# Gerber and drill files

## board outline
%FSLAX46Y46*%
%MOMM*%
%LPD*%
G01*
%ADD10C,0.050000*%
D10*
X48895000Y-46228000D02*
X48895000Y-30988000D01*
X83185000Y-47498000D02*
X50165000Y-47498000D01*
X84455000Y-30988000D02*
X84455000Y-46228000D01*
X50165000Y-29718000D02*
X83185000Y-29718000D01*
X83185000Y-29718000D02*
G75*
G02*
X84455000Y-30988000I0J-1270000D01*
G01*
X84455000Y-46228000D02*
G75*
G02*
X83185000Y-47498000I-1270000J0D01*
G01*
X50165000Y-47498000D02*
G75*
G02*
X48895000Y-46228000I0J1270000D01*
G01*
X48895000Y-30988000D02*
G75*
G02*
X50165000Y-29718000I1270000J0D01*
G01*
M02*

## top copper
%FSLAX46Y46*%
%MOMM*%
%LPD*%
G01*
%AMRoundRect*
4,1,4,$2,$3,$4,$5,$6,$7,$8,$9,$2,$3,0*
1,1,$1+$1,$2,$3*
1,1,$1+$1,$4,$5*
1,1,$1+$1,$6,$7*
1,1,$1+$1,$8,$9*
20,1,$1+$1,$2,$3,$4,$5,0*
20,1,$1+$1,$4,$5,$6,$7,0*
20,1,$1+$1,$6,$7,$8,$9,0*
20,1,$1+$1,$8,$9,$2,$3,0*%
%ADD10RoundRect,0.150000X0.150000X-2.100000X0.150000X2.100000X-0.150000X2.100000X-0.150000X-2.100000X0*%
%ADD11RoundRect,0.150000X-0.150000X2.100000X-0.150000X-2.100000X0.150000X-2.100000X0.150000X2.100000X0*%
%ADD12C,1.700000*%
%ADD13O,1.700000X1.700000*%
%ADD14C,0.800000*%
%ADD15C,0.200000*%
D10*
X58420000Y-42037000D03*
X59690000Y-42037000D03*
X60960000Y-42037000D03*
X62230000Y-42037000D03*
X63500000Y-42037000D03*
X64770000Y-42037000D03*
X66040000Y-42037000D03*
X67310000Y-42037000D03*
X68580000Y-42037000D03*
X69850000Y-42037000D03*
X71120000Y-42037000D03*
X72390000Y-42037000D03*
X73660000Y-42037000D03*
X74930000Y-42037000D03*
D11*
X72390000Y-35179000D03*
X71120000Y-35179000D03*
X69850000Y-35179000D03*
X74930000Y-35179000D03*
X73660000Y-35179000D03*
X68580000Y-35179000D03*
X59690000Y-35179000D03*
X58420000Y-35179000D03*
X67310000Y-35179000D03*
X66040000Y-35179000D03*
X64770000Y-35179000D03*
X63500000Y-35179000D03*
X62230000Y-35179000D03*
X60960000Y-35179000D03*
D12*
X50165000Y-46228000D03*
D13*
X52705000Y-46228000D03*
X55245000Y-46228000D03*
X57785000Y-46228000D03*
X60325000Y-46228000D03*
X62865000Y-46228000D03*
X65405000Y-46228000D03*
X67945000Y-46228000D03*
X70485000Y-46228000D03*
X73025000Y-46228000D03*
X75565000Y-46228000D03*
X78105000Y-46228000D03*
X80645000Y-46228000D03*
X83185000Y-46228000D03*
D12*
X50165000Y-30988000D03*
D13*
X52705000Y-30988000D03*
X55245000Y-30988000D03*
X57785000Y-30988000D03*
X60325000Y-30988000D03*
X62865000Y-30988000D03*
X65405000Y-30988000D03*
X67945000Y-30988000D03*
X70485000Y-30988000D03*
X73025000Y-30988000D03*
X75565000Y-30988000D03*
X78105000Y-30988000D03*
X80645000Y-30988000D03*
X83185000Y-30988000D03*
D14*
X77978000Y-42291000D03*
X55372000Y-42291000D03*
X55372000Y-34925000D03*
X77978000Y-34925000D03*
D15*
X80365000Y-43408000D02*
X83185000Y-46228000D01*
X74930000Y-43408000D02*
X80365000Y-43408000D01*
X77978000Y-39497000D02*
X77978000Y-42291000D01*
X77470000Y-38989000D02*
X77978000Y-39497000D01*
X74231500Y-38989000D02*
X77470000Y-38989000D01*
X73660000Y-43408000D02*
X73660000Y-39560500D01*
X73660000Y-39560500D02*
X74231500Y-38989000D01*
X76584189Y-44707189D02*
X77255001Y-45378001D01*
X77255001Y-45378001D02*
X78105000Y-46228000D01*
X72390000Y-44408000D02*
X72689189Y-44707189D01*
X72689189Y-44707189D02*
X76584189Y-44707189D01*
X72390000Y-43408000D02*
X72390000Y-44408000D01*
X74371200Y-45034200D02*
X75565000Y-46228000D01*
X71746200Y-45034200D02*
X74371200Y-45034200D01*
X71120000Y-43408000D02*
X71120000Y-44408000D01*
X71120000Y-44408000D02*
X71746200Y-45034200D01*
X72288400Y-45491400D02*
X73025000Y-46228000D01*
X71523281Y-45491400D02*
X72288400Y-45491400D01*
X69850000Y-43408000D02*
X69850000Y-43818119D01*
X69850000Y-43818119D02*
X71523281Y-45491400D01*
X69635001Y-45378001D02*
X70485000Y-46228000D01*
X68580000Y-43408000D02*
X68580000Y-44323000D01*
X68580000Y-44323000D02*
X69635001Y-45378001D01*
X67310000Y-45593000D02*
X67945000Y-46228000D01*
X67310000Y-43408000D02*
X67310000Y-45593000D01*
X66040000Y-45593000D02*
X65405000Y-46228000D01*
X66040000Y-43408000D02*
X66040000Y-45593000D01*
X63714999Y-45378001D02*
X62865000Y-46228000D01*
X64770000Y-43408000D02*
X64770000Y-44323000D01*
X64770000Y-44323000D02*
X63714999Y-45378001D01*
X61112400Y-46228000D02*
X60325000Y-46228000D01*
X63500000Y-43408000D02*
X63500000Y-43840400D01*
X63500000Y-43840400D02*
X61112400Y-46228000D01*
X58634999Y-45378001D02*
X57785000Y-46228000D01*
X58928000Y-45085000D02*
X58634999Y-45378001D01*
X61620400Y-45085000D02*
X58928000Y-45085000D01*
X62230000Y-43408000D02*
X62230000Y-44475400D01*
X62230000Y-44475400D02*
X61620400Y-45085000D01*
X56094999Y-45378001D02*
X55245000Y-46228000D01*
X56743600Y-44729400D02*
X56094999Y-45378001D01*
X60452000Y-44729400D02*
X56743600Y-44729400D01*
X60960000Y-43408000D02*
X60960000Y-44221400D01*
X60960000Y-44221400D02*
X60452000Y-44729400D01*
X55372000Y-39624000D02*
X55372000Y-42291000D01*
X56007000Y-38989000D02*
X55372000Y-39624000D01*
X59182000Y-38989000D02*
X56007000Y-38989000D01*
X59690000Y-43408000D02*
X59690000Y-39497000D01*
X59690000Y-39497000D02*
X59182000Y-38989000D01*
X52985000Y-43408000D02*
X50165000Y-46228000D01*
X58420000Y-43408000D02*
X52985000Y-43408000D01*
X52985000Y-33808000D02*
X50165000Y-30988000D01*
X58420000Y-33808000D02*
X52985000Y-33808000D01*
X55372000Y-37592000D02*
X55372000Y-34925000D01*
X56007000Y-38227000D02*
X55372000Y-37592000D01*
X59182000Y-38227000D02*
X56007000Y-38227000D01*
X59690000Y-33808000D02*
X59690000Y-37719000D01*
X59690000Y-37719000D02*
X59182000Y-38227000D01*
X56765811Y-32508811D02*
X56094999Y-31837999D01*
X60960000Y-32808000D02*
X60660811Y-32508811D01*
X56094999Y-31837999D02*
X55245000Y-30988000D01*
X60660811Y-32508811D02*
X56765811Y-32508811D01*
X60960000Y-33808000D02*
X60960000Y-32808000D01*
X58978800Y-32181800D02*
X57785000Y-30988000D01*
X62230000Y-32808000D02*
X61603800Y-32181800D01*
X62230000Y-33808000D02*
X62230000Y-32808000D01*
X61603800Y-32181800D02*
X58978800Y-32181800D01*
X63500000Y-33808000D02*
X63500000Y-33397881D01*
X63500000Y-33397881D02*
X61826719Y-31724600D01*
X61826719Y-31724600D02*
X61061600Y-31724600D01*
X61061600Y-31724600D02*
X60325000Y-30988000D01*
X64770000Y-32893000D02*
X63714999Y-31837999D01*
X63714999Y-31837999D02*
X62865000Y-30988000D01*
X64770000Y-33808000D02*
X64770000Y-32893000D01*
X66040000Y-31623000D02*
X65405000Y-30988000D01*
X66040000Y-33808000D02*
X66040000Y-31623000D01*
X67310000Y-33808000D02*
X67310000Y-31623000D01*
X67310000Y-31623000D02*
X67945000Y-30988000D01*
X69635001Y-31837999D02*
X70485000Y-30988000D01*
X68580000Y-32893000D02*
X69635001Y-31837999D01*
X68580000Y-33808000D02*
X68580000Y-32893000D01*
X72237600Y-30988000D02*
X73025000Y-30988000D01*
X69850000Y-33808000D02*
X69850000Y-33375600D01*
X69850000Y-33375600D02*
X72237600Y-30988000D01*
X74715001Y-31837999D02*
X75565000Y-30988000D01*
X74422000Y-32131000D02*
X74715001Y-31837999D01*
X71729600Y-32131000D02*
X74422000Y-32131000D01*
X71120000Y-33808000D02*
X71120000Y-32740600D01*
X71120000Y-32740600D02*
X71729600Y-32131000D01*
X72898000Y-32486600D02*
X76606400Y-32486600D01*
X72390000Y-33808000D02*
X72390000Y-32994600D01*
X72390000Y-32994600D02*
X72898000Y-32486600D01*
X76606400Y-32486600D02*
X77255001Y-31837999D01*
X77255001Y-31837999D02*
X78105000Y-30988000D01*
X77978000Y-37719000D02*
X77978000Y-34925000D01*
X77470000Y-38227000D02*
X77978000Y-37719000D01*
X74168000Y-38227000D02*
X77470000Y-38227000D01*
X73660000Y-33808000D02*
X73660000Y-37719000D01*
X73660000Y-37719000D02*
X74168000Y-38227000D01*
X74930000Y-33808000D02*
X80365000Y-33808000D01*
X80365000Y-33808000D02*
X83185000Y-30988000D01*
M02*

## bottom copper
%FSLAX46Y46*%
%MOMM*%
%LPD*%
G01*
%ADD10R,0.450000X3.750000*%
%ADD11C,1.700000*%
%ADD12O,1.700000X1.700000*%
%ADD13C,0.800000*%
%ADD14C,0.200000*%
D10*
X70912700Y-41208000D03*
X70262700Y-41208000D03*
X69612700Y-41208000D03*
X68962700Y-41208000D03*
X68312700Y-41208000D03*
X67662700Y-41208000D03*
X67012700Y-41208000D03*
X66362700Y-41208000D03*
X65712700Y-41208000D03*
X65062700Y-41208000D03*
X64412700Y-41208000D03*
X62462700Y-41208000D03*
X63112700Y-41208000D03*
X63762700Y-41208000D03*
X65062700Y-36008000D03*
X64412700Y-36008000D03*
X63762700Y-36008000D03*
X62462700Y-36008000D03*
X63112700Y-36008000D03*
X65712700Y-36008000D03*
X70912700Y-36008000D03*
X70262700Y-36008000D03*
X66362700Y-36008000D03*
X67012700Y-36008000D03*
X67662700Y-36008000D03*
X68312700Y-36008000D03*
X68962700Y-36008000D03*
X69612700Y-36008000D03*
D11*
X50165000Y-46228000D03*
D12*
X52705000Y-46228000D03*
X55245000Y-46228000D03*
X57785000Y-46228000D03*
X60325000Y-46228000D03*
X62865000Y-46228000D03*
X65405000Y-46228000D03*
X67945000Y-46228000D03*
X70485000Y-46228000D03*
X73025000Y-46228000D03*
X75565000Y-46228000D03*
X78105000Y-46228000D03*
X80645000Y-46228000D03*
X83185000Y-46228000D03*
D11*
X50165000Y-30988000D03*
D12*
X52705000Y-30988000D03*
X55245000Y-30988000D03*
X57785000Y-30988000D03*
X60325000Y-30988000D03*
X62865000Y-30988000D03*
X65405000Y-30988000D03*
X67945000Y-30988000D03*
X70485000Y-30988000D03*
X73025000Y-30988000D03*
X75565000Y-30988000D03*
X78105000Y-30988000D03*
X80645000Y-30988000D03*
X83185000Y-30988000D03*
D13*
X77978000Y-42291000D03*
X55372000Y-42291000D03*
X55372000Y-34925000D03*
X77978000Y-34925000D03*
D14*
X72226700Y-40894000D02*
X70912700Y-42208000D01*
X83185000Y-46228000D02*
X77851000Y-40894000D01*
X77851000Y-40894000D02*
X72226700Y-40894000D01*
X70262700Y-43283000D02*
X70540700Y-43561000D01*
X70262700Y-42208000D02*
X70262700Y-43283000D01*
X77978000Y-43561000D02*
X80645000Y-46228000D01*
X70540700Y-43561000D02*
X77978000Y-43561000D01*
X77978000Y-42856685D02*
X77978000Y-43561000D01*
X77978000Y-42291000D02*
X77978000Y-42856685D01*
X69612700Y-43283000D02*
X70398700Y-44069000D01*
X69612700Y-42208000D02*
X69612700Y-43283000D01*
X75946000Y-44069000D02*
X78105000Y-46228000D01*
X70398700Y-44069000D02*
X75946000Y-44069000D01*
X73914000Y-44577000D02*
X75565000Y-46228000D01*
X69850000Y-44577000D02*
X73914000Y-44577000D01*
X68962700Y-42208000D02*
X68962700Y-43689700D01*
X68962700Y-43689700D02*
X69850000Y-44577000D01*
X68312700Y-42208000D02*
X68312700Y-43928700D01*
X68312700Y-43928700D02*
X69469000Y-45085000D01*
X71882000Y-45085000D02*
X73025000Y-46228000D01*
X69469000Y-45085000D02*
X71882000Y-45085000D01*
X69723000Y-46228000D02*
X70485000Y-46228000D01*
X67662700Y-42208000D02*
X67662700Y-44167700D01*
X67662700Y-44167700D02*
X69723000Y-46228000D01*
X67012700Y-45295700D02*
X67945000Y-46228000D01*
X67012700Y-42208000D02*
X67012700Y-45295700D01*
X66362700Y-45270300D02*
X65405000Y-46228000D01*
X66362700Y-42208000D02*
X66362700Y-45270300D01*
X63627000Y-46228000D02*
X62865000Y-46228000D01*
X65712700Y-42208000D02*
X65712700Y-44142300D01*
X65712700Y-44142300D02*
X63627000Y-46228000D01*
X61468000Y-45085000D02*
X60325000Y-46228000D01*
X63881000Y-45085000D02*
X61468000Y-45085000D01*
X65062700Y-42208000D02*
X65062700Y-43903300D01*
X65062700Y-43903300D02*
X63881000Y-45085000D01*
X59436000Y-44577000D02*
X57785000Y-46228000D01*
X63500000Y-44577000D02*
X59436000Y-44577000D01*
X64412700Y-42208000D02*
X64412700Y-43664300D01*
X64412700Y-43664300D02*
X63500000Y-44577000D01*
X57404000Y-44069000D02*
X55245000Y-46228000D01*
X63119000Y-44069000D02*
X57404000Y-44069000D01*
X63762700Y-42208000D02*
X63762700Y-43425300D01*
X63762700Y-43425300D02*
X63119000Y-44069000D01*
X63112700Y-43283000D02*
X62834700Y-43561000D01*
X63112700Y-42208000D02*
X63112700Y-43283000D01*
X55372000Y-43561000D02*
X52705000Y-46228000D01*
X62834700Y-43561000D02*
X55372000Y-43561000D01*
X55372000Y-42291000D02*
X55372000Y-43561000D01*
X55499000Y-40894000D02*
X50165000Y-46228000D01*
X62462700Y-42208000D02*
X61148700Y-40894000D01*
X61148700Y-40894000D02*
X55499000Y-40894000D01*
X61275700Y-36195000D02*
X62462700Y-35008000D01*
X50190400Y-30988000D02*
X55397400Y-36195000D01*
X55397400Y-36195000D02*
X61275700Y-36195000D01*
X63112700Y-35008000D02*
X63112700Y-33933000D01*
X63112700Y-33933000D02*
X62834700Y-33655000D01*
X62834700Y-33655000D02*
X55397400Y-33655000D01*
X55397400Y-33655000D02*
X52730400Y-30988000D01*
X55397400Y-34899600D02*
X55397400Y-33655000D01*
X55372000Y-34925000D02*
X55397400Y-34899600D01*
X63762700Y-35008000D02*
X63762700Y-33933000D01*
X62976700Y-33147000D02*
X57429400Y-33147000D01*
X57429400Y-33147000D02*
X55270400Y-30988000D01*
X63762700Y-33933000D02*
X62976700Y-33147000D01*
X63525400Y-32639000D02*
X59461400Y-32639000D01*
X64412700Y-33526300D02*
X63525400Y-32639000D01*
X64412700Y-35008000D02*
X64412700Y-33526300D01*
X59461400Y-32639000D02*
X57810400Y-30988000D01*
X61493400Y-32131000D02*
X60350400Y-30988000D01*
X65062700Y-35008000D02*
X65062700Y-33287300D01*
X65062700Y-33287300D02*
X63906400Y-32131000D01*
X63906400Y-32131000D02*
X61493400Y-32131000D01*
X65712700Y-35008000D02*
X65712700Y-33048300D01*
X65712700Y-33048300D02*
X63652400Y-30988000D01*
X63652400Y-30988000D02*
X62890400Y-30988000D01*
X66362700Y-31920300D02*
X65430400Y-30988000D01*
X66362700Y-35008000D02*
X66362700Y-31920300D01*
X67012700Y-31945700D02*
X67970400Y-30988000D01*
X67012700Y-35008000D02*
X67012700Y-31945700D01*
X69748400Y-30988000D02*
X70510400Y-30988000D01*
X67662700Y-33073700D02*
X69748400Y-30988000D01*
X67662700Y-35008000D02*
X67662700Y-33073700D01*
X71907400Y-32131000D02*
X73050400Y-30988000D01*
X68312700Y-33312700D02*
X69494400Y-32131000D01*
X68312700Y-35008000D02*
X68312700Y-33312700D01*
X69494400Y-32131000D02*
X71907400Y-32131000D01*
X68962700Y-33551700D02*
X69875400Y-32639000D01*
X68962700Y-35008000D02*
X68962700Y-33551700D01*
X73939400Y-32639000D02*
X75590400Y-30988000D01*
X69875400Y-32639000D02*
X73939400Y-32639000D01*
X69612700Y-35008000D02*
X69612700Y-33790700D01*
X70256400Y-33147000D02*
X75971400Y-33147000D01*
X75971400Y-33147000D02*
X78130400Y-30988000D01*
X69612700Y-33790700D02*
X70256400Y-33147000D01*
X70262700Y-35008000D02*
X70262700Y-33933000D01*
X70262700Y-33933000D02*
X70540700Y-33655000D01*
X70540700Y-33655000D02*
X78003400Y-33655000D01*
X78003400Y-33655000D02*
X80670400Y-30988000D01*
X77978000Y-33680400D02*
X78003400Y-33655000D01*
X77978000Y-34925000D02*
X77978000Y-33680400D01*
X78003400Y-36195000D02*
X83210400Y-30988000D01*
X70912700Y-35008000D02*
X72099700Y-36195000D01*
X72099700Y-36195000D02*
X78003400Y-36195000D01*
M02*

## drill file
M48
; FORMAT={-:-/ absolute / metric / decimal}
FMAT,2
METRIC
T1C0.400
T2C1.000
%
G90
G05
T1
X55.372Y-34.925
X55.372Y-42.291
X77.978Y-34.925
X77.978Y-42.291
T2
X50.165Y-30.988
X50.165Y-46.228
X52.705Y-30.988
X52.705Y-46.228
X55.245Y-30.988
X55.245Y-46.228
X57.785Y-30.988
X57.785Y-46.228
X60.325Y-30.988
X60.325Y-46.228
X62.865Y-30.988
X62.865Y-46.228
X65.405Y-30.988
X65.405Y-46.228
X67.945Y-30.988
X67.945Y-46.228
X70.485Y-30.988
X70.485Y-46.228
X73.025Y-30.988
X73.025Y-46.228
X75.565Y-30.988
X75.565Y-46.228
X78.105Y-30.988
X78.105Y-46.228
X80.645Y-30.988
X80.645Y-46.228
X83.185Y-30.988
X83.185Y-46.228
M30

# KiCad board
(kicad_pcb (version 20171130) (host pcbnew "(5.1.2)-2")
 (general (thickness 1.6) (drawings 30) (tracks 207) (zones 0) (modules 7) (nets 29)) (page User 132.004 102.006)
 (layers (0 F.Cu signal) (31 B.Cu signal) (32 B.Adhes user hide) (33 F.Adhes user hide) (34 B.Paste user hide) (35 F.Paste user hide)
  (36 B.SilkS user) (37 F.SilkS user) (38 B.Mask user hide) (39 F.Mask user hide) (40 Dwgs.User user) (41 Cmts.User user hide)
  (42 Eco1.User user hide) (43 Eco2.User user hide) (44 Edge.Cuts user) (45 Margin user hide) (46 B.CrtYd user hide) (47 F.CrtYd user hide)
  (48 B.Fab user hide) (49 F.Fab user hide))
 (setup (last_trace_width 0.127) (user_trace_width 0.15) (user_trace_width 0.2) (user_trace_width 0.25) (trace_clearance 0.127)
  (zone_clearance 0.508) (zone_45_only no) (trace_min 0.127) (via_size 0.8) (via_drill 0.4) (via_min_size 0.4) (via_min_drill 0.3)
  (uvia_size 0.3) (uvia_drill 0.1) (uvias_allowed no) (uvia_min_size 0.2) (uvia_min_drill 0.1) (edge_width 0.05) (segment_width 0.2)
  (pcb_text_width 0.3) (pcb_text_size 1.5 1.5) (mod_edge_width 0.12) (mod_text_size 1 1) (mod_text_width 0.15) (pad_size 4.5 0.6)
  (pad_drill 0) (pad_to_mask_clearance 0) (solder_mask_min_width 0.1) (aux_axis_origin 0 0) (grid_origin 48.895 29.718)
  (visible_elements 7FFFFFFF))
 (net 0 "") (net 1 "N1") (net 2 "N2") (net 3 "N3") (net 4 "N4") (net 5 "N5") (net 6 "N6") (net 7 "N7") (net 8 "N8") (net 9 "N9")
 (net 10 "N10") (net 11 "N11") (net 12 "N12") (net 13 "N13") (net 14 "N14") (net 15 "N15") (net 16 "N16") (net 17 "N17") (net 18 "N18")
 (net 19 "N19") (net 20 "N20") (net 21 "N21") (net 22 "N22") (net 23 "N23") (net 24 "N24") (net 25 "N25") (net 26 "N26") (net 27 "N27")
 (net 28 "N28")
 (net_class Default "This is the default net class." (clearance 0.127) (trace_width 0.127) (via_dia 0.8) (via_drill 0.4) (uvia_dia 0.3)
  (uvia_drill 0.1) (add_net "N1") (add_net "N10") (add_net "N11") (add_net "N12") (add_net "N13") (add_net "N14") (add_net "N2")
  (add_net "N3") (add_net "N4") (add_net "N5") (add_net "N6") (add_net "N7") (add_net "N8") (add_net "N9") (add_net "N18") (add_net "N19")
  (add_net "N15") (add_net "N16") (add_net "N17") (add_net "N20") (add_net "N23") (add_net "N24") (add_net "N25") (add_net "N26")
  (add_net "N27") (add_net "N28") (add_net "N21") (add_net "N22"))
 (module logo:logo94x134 (layer B.Cu) (at 79.502 38.608 180)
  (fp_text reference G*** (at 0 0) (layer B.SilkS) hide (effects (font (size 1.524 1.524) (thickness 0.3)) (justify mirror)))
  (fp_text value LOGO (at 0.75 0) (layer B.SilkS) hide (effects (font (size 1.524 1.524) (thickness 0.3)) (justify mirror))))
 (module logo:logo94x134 (layer F.Cu) (at 52.705 38.608)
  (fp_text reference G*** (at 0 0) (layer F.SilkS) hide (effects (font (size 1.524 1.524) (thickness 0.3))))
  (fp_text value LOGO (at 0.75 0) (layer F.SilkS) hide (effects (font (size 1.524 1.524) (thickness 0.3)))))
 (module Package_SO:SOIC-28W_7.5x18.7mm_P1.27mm (layer F.Cu) (at 66.675 38.608 90)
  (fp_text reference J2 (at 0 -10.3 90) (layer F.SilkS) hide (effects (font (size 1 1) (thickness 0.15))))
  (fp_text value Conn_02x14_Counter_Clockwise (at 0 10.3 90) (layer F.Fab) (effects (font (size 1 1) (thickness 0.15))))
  (pad 1 smd roundrect (at -3.429 -8.255 90) (size 4.5 0.6) (layers F.Cu F.Paste F.Mask) (roundrect_rratio 0.25) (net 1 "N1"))
  (pad 2 smd roundrect (at -3.429 -6.985 90) (size 4.5 0.6) (layers F.Cu F.Paste F.Mask) (roundrect_rratio 0.25) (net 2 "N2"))
  (pad 3 smd roundrect (at -3.429 -5.715 90) (size 4.5 0.6) (layers F.Cu F.Paste F.Mask) (roundrect_rratio 0.25) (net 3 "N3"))
  (pad 4 smd roundrect (at -3.429 -4.445 90) (size 4.5 0.6) (layers F.Cu F.Paste F.Mask) (roundrect_rratio 0.25) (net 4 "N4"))
  (pad 5 smd roundrect (at -3.429 -3.175 90) (size 4.5 0.6) (layers F.Cu F.Paste F.Mask) (roundrect_rratio 0.25) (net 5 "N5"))
  (pad 6 smd roundrect (at -3.429 -1.905 90) (size 4.5 0.6) (layers F.Cu F.Paste F.Mask) (roundrect_rratio 0.25) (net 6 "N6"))
  (pad 7 smd roundrect (at -3.429 -0.635 90) (size 4.5 0.6) (layers F.Cu F.Paste F.Mask) (roundrect_rratio 0.25) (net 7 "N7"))
  (pad 8 smd roundrect (at -3.429 0.635 90) (size 4.5 0.6) (layers F.Cu F.Paste F.Mask) (roundrect_rratio 0.25) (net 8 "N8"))
  (pad 9 smd roundrect (at -3.429 1.905 90) (size 4.5 0.6) (layers F.Cu F.Paste F.Mask) (roundrect_rratio 0.25) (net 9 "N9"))
  (pad 10 smd roundrect (at -3.429 3.175 90) (size 4.5 0.6) (layers F.Cu F.Paste F.Mask) (roundrect_rratio 0.25) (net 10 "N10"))
  (pad 11 smd roundrect (at -3.429 4.445 90) (size 4.5 0.6) (layers F.Cu F.Paste F.Mask) (roundrect_rratio 0.25) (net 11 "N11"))
  (pad 12 smd roundrect (at -3.429 5.715 90) (size 4.5 0.6) (layers F.Cu F.Paste F.Mask) (roundrect_rratio 0.25) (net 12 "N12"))
  (pad 13 smd roundrect (at -3.429 6.985 90) (size 4.5 0.6) (layers F.Cu F.Paste F.Mask) (roundrect_rratio 0.25) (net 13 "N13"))
  (pad 14 smd roundrect (at -3.429 8.255 90) (size 4.5 0.6) (layers F.Cu F.Paste F.Mask) (roundrect_rratio 0.25) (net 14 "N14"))
  (pad 17 smd roundrect (at 3.429 5.715 270) (size 4.5 0.6) (layers F.Cu F.Paste F.Mask) (roundrect_rratio 0.25) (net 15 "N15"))
  (pad 18 smd roundrect (at 3.429 4.445 270) (size 4.5 0.6) (layers F.Cu F.Paste F.Mask) (roundrect_rratio 0.25) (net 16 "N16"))
  (pad 19 smd roundrect (at 3.429 3.175 270) (size 4.5 0.6) (layers F.Cu F.Paste F.Mask) (roundrect_rratio 0.25) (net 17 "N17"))
  (pad 15 smd roundrect (at 3.429 8.255 270) (size 4.5 0.6) (layers F.Cu F.Paste F.Mask) (roundrect_rratio 0.25) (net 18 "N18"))
  (pad 16 smd roundrect (at 3.429 6.985 270) (size 4.5 0.6) (layers F.Cu F.Paste F.Mask) (roundrect_rratio 0.25) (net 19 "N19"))
  (pad 20 smd roundrect (at 3.429 1.905 270) (size 4.5 0.6) (layers F.Cu F.Paste F.Mask) (roundrect_rratio 0.25) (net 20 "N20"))
  (pad 27 smd roundrect (at 3.429 -6.985 270) (size 4.5 0.6) (layers F.Cu F.Paste F.Mask) (roundrect_rratio 0.25) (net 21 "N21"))
  (pad 8 smd roundrect (at 3.429 -8.255 270) (size 4.5 0.6) (layers F.Cu F.Paste F.Mask) (roundrect_rratio 0.25) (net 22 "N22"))
  (pad 21 smd roundrect (at 3.429 0.635 270) (size 4.5 0.6) (layers F.Cu F.Paste F.Mask) (roundrect_rratio 0.25) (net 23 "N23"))
  (pad 22 smd roundrect (at 3.429 -0.635 270) (size 4.5 0.6) (layers F.Cu F.Paste F.Mask) (roundrect_rratio 0.25) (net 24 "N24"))
  (pad 23 smd roundrect (at 3.429 -1.905 270) (size 4.5 0.6) (layers F.Cu F.Paste F.Mask) (roundrect_rratio 0.25) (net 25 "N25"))
  (pad 24 smd roundrect (at 3.429 -3.175 270) (size 4.5 0.6) (layers F.Cu F.Paste F.Mask) (roundrect_rratio 0.25) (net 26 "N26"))
  (pad 25 smd roundrect (at 3.429 -4.445 270) (size 4.5 0.6) (layers F.Cu F.Paste F.Mask) (roundrect_rratio 0.25) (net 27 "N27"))
  (pad 26 smd roundrect (at 3.429 -5.715 270) (size 4.5 0.6) (layers F.Cu F.Paste F.Mask) (roundrect_rratio 0.25) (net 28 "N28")))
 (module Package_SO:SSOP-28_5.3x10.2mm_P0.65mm (layer B.Cu) (at 66.6877 38.608 90)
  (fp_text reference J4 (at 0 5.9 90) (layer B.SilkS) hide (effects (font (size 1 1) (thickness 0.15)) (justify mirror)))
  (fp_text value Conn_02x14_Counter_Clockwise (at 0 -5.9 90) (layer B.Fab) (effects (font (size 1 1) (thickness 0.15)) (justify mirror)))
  (pad 1 smd rect (at -2.6 4.225 90) (size 3.75 0.45) (layers B.Cu B.Paste B.Mask) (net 14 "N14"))
  (pad 2 smd rect (at -2.6 3.575 90) (size 3.75 0.45) (layers B.Cu B.Paste B.Mask) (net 13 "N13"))
  (pad 3 smd rect (at -2.6 2.925 90) (size 3.75 0.45) (layers B.Cu B.Paste B.Mask) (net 12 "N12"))
  (pad 4 smd rect (at -2.6 2.275 90) (size 3.75 0.45) (layers B.Cu B.Paste B.Mask) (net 11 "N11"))
  (pad 5 smd rect (at -2.6 1.625 90) (size 3.75 0.45) (layers B.Cu B.Paste B.Mask) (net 10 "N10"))
  (pad 6 smd rect (at -2.6 0.975 90) (size 3.75 0.45) (layers B.Cu B.Paste B.Mask) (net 9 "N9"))
  (pad 7 smd rect (at -2.6 0.325 90) (size 3.75 0.45) (layers B.Cu B.Paste B.Mask) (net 8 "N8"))
  (pad 8 smd rect (at -2.6 -0.325 90) (size 3.75 0.45) (layers B.Cu B.Paste B.Mask) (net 7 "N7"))
  (pad 9 smd rect (at -2.6 -0.975 90) (size 3.75 0.45) (layers B.Cu B.Paste B.Mask) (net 6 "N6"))
  (pad 10 smd rect (at -2.6 -1.625 90) (size 3.75 0.45) (layers B.Cu B.Paste B.Mask) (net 5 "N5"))
  (pad 11 smd rect (at -2.6 -2.275 90) (size 3.75 0.45) (layers B.Cu B.Paste B.Mask) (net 4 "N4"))
  (pad 14 smd rect (at -2.6 -4.225 90) (size 3.75 0.45) (layers B.Cu B.Paste B.Mask) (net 1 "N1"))
  (pad 13 smd rect (at -2.6 -3.575 90) (size 3.75 0.45) (layers B.Cu B.Paste B.Mask) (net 2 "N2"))
  (pad 12 smd rect (at -2.6 -2.925 90) (size 3.75 0.45) (layers B.Cu B.Paste B.Mask) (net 3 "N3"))
  (pad 19 smd rect (at 2.6 -1.625 270) (size 3.75 0.45) (layers B.Cu B.Paste B.Mask) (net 26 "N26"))
  (pad 18 smd rect (at 2.6 -2.275 270) (size 3.75 0.45) (layers B.Cu B.Paste B.Mask) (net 27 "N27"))
  (pad 17 smd rect (at 2.6 -2.925 270) (size 3.75 0.45) (layers B.Cu B.Paste B.Mask) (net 28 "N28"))
  (pad 15 smd rect (at 2.6 -4.225 270) (size 3.75 0.45) (layers B.Cu B.Paste B.Mask) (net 22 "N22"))
  (pad 16 smd rect (at 2.6 -3.575 270) (size 3.75 0.45) (layers B.Cu B.Paste B.Mask) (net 21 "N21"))
  (pad 20 smd rect (at 2.6 -0.975 270) (size 3.75 0.45) (layers B.Cu B.Paste B.Mask) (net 25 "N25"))
  (pad 28 smd rect (at 2.6 4.225 270) (size 3.75 0.45) (layers B.Cu B.Paste B.Mask) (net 18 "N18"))
  (pad 27 smd rect (at 2.6 3.575 270) (size 3.75 0.45) (layers B.Cu B.Paste B.Mask) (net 19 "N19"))
  (pad 21 smd rect (at 2.6 -0.325 270) (size 3.75 0.45) (layers B.Cu B.Paste B.Mask) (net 24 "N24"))
  (pad 22 smd rect (at 2.6 0.325 270) (size 3.75 0.45) (layers B.Cu B.Paste B.Mask) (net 23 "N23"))
  (pad 23 smd rect (at 2.6 0.975 270) (size 3.75 0.45) (layers B.Cu B.Paste B.Mask) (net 20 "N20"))
  (pad 24 smd rect (at 2.6 1.625 270) (size 3.75 0.45) (layers B.Cu B.Paste B.Mask) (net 17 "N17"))
  (pad 25 smd rect (at 2.6 2.275 270) (size 3.75 0.45) (layers B.Cu B.Paste B.Mask) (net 16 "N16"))
  (pad 26 smd rect (at 2.6 2.925 270) (size 3.75 0.45) (layers B.Cu B.Paste B.Mask) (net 15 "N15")))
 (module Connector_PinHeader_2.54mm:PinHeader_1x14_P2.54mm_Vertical (layer B.Cu) (at 50.165 46.228 270)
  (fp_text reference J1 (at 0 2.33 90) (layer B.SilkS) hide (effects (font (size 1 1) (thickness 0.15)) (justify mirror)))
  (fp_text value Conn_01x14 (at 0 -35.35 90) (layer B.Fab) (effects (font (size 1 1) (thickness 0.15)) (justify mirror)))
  (pad 1 thru_hole circle (at 0 0 270) (size 1.7 1.7) (drill 1) (layers *.Cu *.Mask) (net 1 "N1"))
  (pad 2 thru_hole oval (at 0 -2.54 270) (size 1.7 1.7) (drill 1) (layers *.Cu *.Mask) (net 2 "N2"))
  (pad 3 thru_hole oval (at 0 -5.08 270) (size 1.7 1.7) (drill 1) (layers *.Cu *.Mask) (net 3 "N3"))
  (pad 4 thru_hole oval (at 0 -7.62 270) (size 1.7 1.7) (drill 1) (layers *.Cu *.Mask) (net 4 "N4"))
  (pad 5 thru_hole oval (at 0 -10.16 270) (size 1.7 1.7) (drill 1) (layers *.Cu *.Mask) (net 5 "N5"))
  (pad 6 thru_hole oval (at 0 -12.7 270) (size 1.7 1.7) (drill 1) (layers *.Cu *.Mask) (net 6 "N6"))
  (pad 7 thru_hole oval (at 0 -15.24 270) (size 1.7 1.7) (drill 1) (layers *.Cu *.Mask) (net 7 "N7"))
  (pad 8 thru_hole oval (at 0 -17.78 270) (size 1.7 1.7) (drill 1) (layers *.Cu *.Mask) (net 8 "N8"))
  (pad 9 thru_hole oval (at 0 -20.32 270) (size 1.7 1.7) (drill 1) (layers *.Cu *.Mask) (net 9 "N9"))
  (pad 10 thru_hole oval (at 0 -22.86 270) (size 1.7 1.7) (drill 1) (layers *.Cu *.Mask) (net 10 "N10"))
  (pad 11 thru_hole oval (at 0 -25.4 270) (size 1.7 1.7) (drill 1) (layers *.Cu *.Mask) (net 11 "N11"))
  (pad 12 thru_hole oval (at 0 -27.94 270) (size 1.7 1.7) (drill 1) (layers *.Cu *.Mask) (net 12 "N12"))
  (pad 13 thru_hole oval (at 0 -30.48 270) (size 1.7 1.7) (drill 1) (layers *.Cu *.Mask) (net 13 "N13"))
  (pad 14 thru_hole oval (at 0 -33.02 270) (size 1.7 1.7) (drill 1) (layers *.Cu *.Mask) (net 14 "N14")))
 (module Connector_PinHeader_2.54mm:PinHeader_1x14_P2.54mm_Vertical (layer B.Cu) (at 50.165 30.988 270)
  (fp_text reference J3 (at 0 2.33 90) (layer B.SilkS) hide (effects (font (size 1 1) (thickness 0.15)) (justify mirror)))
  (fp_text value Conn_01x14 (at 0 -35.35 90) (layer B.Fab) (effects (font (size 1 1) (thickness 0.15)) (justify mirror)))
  (pad 1 thru_hole circle (at 0 0 270) (size 1.7 1.7) (drill 1) (layers *.Cu *.Mask) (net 22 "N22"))
  (pad 2 thru_hole oval (at 0 -2.54 270) (size 1.7 1.7) (drill 1) (layers *.Cu *.Mask) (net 21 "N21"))
  (pad 3 thru_hole oval (at 0 -5.08 270) (size 1.7 1.7) (drill 1) (layers *.Cu *.Mask) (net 28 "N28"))
  (pad 4 thru_hole oval (at 0 -7.62 270) (size 1.7 1.7) (drill 1) (layers *.Cu *.Mask) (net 27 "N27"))
  (pad 5 thru_hole oval (at 0 -10.16 270) (size 1.7 1.7) (drill 1) (layers *.Cu *.Mask) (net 26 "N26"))
  (pad 6 thru_hole oval (at 0 -12.7 270) (size 1.7 1.7) (drill 1) (layers *.Cu *.Mask) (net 25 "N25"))
  (pad 7 thru_hole oval (at 0 -15.24 270) (size 1.7 1.7) (drill 1) (layers *.Cu *.Mask) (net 24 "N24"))
  (pad 8 thru_hole oval (at 0 -17.78 270) (size 1.7 1.7) (drill 1) (layers *.Cu *.Mask) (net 23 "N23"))
  (pad 9 thru_hole oval (at 0 -20.32 270) (size 1.7 1.7) (drill 1) (layers *.Cu *.Mask) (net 20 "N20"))
  (pad 10 thru_hole oval (at 0 -22.86 270) (size 1.7 1.7) (drill 1) (layers *.Cu *.Mask) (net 17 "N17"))
  (pad 11 thru_hole oval (at 0 -25.4 270) (size 1.7 1.7) (drill 1) (layers *.Cu *.Mask) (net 16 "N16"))
  (pad 12 thru_hole oval (at 0 -27.94 270) (size 1.7 1.7) (drill 1) (layers *.Cu *.Mask) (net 15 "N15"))
  (pad 13 thru_hole oval (at 0 -30.48 270) (size 1.7 1.7) (drill 1) (layers *.Cu *.Mask) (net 19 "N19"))
  (pad 14 thru_hole oval (at 0 -33.02 270) (size 1.7 1.7) (drill 1) (layers *.Cu *.Mask) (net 18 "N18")))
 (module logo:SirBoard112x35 (layer B.Cu) (at 58.42 38.608 90)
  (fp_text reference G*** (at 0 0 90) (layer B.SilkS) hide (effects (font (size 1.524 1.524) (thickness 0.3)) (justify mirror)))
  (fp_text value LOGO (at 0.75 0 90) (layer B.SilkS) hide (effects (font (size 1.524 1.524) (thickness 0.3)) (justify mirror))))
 (gr_line (start 48.895 46.228) (end 48.895 30.988) (layer Edge.Cuts) (width 0.05))
 (gr_line (start 83.185 47.498) (end 50.165 47.498) (layer Edge.Cuts) (width 0.05))
 (gr_line (start 84.455 30.988) (end 84.455 46.228) (layer Edge.Cuts) (width 0.05))
 (gr_line (start 50.165 29.718) (end 83.185 29.718) (layer Edge.Cuts) (width 0.05))
 (gr_arc (start 83.185 30.988) (end 84.455 30.988) (angle -90) (layer Edge.Cuts) (width 0.05))
 (gr_arc (start 83.185 46.228) (end 83.185 47.498) (angle -90) (layer Edge.Cuts) (width 0.05))
 (gr_arc (start 50.165 46.228) (end 48.895 46.228) (angle -90) (layer Edge.Cuts) (width 0.05))
 (gr_arc (start 50.165 30.988) (end 50.165 29.718) (angle -90) (layer Edge.Cuts) (width 0.05))
 (segment (start 80.365 43.408) (end 83.185 46.228) (width 0.2) (layer F.Cu) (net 14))
 (segment (start 74.93 43.408) (end 80.365 43.408) (width 0.2) (layer F.Cu) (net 14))
 (segment (start 72.2267 40.894) (end 70.9127 42.208) (width 0.2) (layer B.Cu) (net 14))
 (segment (start 83.185 46.228) (end 77.851 40.894) (width 0.2) (layer B.Cu) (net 14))
 (segment (start 77.851 40.894) (end 72.2267 40.894) (width 0.2) (layer B.Cu) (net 14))
 (segment (start 70.2627 43.283) (end 70.5407 43.561) (width 0.2) (layer B.Cu) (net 13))
 (segment (start 70.2627 42.208) (end 70.2627 43.283) (width 0.2) (layer B.Cu) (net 13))
 (segment (start 77.978 43.561) (end 80.645 46.228) (width 0.2) (layer B.Cu) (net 13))
 (segment (start 70.5407 43.561) (end 77.978 43.561) (width 0.2) (layer B.Cu) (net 13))
 (via (at 77.978 42.291) (size 0.8) (drill 0.4) (layers F.Cu B.Cu) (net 13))
 (segment (start 77.978 42.856685) (end 77.978 43.561) (width 0.2) (layer B.Cu) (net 13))
 (segment (start 77.978 42.291) (end 77.978 42.856685) (width 0.2) (layer B.Cu) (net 13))
 (segment (start 77.978 39.497) (end 77.978 42.291) (width 0.2) (layer F.Cu) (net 13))
 (segment (start 77.47 38.989) (end 77.978 39.497) (width 0.2) (layer F.Cu) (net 13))
 (segment (start 74.2315 38.989) (end 77.47 38.989) (width 0.2) (layer F.Cu) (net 13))
 (segment (start 73.66 43.408) (end 73.66 39.5605) (width 0.2) (layer F.Cu) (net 13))
 (segment (start 73.66 39.5605) (end 74.2315 38.989) (width 0.2) (layer F.Cu) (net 13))
 (segment (start 69.6127 43.283) (end 70.3987 44.069) (width 0.2) (layer B.Cu) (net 12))
 (segment (start 69.6127 42.208) (end 69.6127 43.283) (width 0.2) (layer B.Cu) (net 12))
 (segment (start 75.946 44.069) (end 78.105 46.228) (width 0.2) (layer B.Cu) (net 12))
 (segment (start 70.3987 44.069) (end 75.946 44.069) (width 0.2) (layer B.Cu) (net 12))
 (segment (start 76.584189 44.707189) (end 77.255001 45.378001) (width 0.2) (layer F.Cu) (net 12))
 (segment (start 77.255001 45.378001) (end 78.105 46.228) (width 0.2) (layer F.Cu) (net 12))
 (segment (start 72.39 44.408) (end 72.689189 44.707189) (width 0.2) (layer F.Cu) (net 12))
 (segment (start 72.689189 44.707189) (end 76.584189 44.707189) (width 0.2) (layer F.Cu) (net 12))
 (segment (start 72.39 43.408) (end 72.39 44.408) (width 0.2) (layer F.Cu) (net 12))
 (segment (start 73.914 44.577) (end 75.565 46.228) (width 0.2) (layer B.Cu) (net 11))
 (segment (start 69.85 44.577) (end 73.914 44.577) (width 0.2) (layer B.Cu) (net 11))
 (segment (start 68.9627 42.208) (end 68.9627 43.6897) (width 0.2) (layer B.Cu) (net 11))
 (segment (start 68.9627 43.6897) (end 69.85 44.577) (width 0.2) (layer B.Cu) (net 11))
 (segment (start 74.3712 45.0342) (end 75.565 46.228) (width 0.2) (layer F.Cu) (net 11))
 (segment (start 71.7462 45.0342) (end 74.3712 45.0342) (width 0.2) (layer F.Cu) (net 11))
 (segment (start 71.12 43.408) (end 71.12 44.408) (width 0.2) (layer F.Cu) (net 11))
 (segment (start 71.12 44.408) (end 71.7462 45.0342) (width 0.2) (layer F.Cu) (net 11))
 (segment (start 68.3127 42.208) (end 68.3127 43.9287) (width 0.2) (layer B.Cu) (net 10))
 (segment (start 68.3127 43.9287) (end 69.469 45.085) (width 0.2) (layer B.Cu) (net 10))
 (segment (start 71.882 45.085) (end 73.025 46.228) (width 0.2) (layer B.Cu) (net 10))
 (segment (start 69.469 45.085) (end 71.882 45.085) (width 0.2) (layer B.Cu) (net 10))
 (segment (start 72.2884 45.4914) (end 73.025 46.228) (width 0.2) (layer F.Cu) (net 10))
 (segment (start 71.523281 45.4914) (end 72.2884 45.4914) (width 0.2) (layer F.Cu) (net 10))
 (segment (start 69.85 43.408) (end 69.85 43.818119) (width 0.2) (layer F.Cu) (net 10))
 (segment (start 69.85 43.818119) (end 71.523281 45.4914) (width 0.2) (layer F.Cu) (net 10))
 (segment (start 69.723 46.228) (end 70.485 46.228) (width 0.2) (layer B.Cu) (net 9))
 (segment (start 67.6627 42.208) (end 67.6627 44.1677) (width 0.2) (layer B.Cu) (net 9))
 (segment (start 67.6627 44.1677) (end 69.723 46.228) (width 0.2) (layer B.Cu) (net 9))
 (segment (start 69.635001 45.378001) (end 70.485 46.228) (width 0.2) (layer F.Cu) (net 9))
 (segment (start 68.58 43.408) (end 68.58 44.323) (width 0.2) (layer F.Cu) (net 9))
 (segment (start 68.58 44.323) (end 69.635001 45.378001) (width 0.2) (layer F.Cu) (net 9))
 (segment (start 67.0127 45.2957) (end 67.945 46.228) (width 0.2) (layer B.Cu) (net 8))
 (segment (start 67.0127 42.208) (end 67.0127 45.2957) (width 0.2) (layer B.Cu) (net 8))
 (segment (start 67.31 45.593) (end 67.945 46.228) (width 0.2) (layer F.Cu) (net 8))
 (segment (start 67.31 43.408) (end 67.31 45.593) (width 0.2) (layer F.Cu) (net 8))
 (segment (start 66.3627 45.2703) (end 65.405 46.228) (width 0.2) (layer B.Cu) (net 7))
 (segment (start 66.3627 42.208) (end 66.3627 45.2703) (width 0.2) (layer B.Cu) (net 7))
 (segment (start 66.04 45.593) (end 65.405 46.228) (width 0.2) (layer F.Cu) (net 7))
 (segment (start 66.04 43.408) (end 66.04 45.593) (width 0.2) (layer F.Cu) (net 7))
 (segment (start 63.627 46.228) (end 62.865 46.228) (width 0.2) (layer B.Cu) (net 6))
 (segment (start 65.7127 42.208) (end 65.7127 44.1423) (width 0.2) (layer B.Cu) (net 6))
 (segment (start 65.7127 44.1423) (end 63.627 46.228) (width 0.2) (layer B.Cu) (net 6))
 (segment (start 63.714999 45.378001) (end 62.865 46.228) (width 0.2) (layer F.Cu) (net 6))
 (segment (start 64.77 43.408) (end 64.77 44.323) (width 0.2) (layer F.Cu) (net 6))
 (segment (start 64.77 44.323) (end 63.714999 45.378001) (width 0.2) (layer F.Cu) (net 6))
 (segment (start 61.468 45.085) (end 60.325 46.228) (width 0.2) (layer B.Cu) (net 5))
 (segment (start 63.881 45.085) (end 61.468 45.085) (width 0.2) (layer B.Cu) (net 5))
 (segment (start 65.0627 42.208) (end 65.0627 43.9033) (width 0.2) (layer B.Cu) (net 5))
 (segment (start 65.0627 43.9033) (end 63.881 45.085) (width 0.2) (layer B.Cu) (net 5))
 (segment (start 61.1124 46.228) (end 60.325 46.228) (width 0.2) (layer F.Cu) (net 5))
 (segment (start 63.5 43.408) (end 63.5 43.8404) (width 0.2) (layer F.Cu) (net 5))
 (segment (start 63.5 43.8404) (end 61.1124 46.228) (width 0.2) (layer F.Cu) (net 5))
 (segment (start 59.436 44.577) (end 57.785 46.228) (width 0.2) (layer B.Cu) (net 4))
 (segment (start 63.5 44.577) (end 59.436 44.577) (width 0.2) (layer B.Cu) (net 4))
 (segment (start 64.4127 42.208) (end 64.4127 43.6643) (width 0.2) (layer B.Cu) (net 4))
 (segment (start 64.4127 43.6643) (end 63.5 44.577) (width 0.2) (layer B.Cu) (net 4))
 (segment (start 58.634999 45.378001) (end 57.785 46.228) (width 0.2) (layer F.Cu) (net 4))
 (segment (start 58.928 45.085) (end 58.634999 45.378001) (width 0.2) (layer F.Cu) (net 4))
 (segment (start 61.6204 45.085) (end 58.928 45.085) (width 0.2) (layer F.Cu) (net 4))
 (segment (start 62.23 43.408) (end 62.23 44.4754) (width 0.2) (layer F.Cu) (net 4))
 (segment (start 62.23 44.4754) (end 61.6204 45.085) (width 0.2) (layer F.Cu) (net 4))
 (segment (start 57.404 44.069) (end 55.245 46.228) (width 0.2) (layer B.Cu) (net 3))
 (segment (start 63.119 44.069) (end 57.404 44.069) (width 0.2) (layer B.Cu) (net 3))
 (segment (start 63.7627 42.208) (end 63.7627 43.4253) (width 0.2) (layer B.Cu) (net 3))
 (segment (start 63.7627 43.4253) (end 63.119 44.069) (width 0.2) (layer B.Cu) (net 3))
 (segment (start 56.094999 45.378001) (end 55.245 46.228) (width 0.2) (layer F.Cu) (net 3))
 (segment (start 56.7436 44.7294) (end 56.094999 45.378001) (width 0.2) (layer F.Cu) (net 3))
 (segment (start 60.452 44.7294) (end 56.7436 44.7294) (width 0.2) (layer F.Cu) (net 3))
 (segment (start 60.96 43.408) (end 60.96 44.2214) (width 0.2) (layer F.Cu) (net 3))
 (segment (start 60.96 44.2214) (end 60.452 44.7294) (width 0.2) (layer F.Cu) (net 3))
 (segment (start 63.1127 43.283) (end 62.8347 43.561) (width 0.2) (layer B.Cu) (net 2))
 (segment (start 63.1127 42.208) (end 63.1127 43.283) (width 0.2) (layer B.Cu) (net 2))
 (segment (start 55.372 43.561) (end 52.705 46.228) (width 0.2) (layer B.Cu) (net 2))
 (segment (start 62.8347 43.561) (end 55.372 43.561) (width 0.2) (layer B.Cu) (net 2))
 (via (at 55.372 42.291) (size 0.8) (drill 0.4) (layers F.Cu B.Cu) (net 2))
 (segment (start 55.372 42.291) (end 55.372 43.561) (width 0.2) (layer B.Cu) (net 2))
 (segment (start 55.372 39.624) (end 55.372 42.291) (width 0.2) (layer F.Cu) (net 2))
 (segment (start 56.007 38.989) (end 55.372 39.624) (width 0.2) (layer F.Cu) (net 2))
 (segment (start 59.182 38.989) (end 56.007 38.989) (width 0.2) (layer F.Cu) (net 2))
 (segment (start 59.69 43.408) (end 59.69 39.497) (width 0.2) (layer F.Cu) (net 2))
 (segment (start 59.69 39.497) (end 59.182 38.989) (width 0.2) (layer F.Cu) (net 2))
 (segment (start 52.985 43.408) (end 50.165 46.228) (width 0.2) (layer F.Cu) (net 1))
 (segment (start 58.42 43.408) (end 52.985 43.408) (width 0.2) (layer F.Cu) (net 1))
 (segment (start 55.499 40.894) (end 50.165 46.228) (width 0.2) (layer B.Cu) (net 1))
 (segment (start 62.4627 42.208) (end 61.1487 40.894) (width 0.2) (layer B.Cu) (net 1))
 (segment (start 61.1487 40.894) (end 55.499 40.894) (width 0.2) (layer B.Cu) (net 1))
 (segment (start 52.985 33.808) (end 50.165 30.988) (width 0.2) (layer F.Cu) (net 22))
 (segment (start 61.2757 36.195) (end 62.4627 35.008) (width 0.2) (layer B.Cu) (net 22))
 (segment (start 50.1904 30.988) (end 55.3974 36.195) (width 0.2) (layer B.Cu) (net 22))
 (segment (start 55.3974 36.195) (end 61.2757 36.195) (width 0.2) (layer B.Cu) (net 22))
 (segment (start 58.42 33.808) (end 52.985 33.808) (width 0.2) (layer F.Cu) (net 22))
 (via (at 55.372 34.925) (size 0.8) (drill 0.4) (layers F.Cu B.Cu) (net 21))
 (segment (start 63.1127 35.008) (end 63.1127 33.933) (width 0.2) (layer B.Cu) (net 21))
 (segment (start 63.1127 33.933) (end 62.8347 33.655) (width 0.2) (layer B.Cu) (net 21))
 (segment (start 62.8347 33.655) (end 55.3974 33.655) (width 0.2) (layer B.Cu) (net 21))
 (segment (start 55.3974 33.655) (end 52.7304 30.988) (width 0.2) (layer B.Cu) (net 21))
 (segment (start 55.3974 34.8996) (end 55.3974 33.655) (width 0.2) (layer B.Cu) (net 21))
 (segment (start 55.372 34.925) (end 55.3974 34.8996) (width 0.2) (layer B.Cu) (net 21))
 (segment (start 55.372 37.592) (end 55.372 34.925) (width 0.2) (layer F.Cu) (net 21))
 (segment (start 56.007 38.227) (end 55.372 37.592) (width 0.2) (layer F.Cu) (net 21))
 (segment (start 59.182 38.227) (end 56.007 38.227) (width 0.2) (layer F.Cu) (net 21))
 (segment (start 59.69 33.808) (end 59.69 37.719) (width 0.2) (layer F.Cu) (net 21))
 (segment (start 59.69 37.719) (end 59.182 38.227) (width 0.2) (layer F.Cu) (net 21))
 (segment (start 56.765811 32.508811) (end 56.094999 31.837999) (width 0.2) (layer F.Cu) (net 28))
 (segment (start 60.96 32.808) (end 60.660811 32.508811) (width 0.2) (layer F.Cu) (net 28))
 (segment (start 56.094999 31.837999) (end 55.245 30.988) (width 0.2) (layer F.Cu) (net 28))
 (segment (start 60.660811 32.508811) (end 56.765811 32.508811) (width 0.2) (layer F.Cu) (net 28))
 (segment (start 60.96 33.808) (end 60.96 32.808) (width 0.2) (layer F.Cu) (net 28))
 (segment (start 63.7627 35.008) (end 63.7627 33.933) (width 0.2) (layer B.Cu) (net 28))
 (segment (start 62.9767 33.147) (end 57.4294 33.147) (width 0.2) (layer B.Cu) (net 28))
 (segment (start 57.4294 33.147) (end 55.2704 30.988) (width 0.2) (layer B.Cu) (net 28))
 (segment (start 63.7627 33.933) (end 62.9767 33.147) (width 0.2) (layer B.Cu) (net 28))
 (segment (start 58.9788 32.1818) (end 57.785 30.988) (width 0.2) (layer F.Cu) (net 27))
 (segment (start 62.23 32.808) (end 61.6038 32.1818) (width 0.2) (layer F.Cu) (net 27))
 (segment (start 62.23 33.808) (end 62.23 32.808) (width 0.2) (layer F.Cu) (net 27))
 (segment (start 61.6038 32.1818) (end 58.9788 32.1818) (width 0.2) (layer F.Cu) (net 27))
 (segment (start 63.5254 32.639) (end 59.4614 32.639) (width 0.2) (layer B.Cu) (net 27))
 (segment (start 64.4127 33.5263) (end 63.5254 32.639) (width 0.2) (layer B.Cu) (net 27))
 (segment (start 64.4127 35.008) (end 64.4127 33.5263) (width 0.2) (layer B.Cu) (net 27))
 (segment (start 59.4614 32.639) (end 57.8104 30.988) (width 0.2) (layer B.Cu) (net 27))
 (segment (start 63.5 33.808) (end 63.5 33.397881) (width 0.2) (layer F.Cu) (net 26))
 (segment (start 63.5 33.397881) (end 61.826719 31.7246) (width 0.2) (layer F.Cu) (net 26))
 (segment (start 61.826719 31.7246) (end 61.0616 31.7246) (width 0.2) (layer F.Cu) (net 26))
 (segment (start 61.0616 31.7246) (end 60.325 30.988) (width 0.2) (layer F.Cu) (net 26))
 (segment (start 61.4934 32.131) (end 60.3504 30.988) (width 0.2) (layer B.Cu) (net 26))
 (segment (start 65.0627 35.008) (end 65.0627 33.2873) (width 0.2) (layer B.Cu) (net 26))
 (segment (start 65.0627 33.2873) (end 63.9064 32.131) (width 0.2) (layer B.Cu) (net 26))
 (segment (start 63.9064 32.131) (end 61.4934 32.131) (width 0.2) (layer B.Cu) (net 26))
 (segment (start 64.77 32.893) (end 63.714999 31.837999) (width 0.2) (layer F.Cu) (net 25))
 (segment (start 63.714999 31.837999) (end 62.865 30.988) (width 0.2) (layer F.Cu) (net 25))
 (segment (start 64.77 33.808) (end 64.77 32.893) (width 0.2) (layer F.Cu) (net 25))
 (segment (start 65.7127 35.008) (end 65.7127 33.0483) (width 0.2) (layer B.Cu) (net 25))
 (segment (start 65.7127 33.0483) (end 63.6524 30.988) (width 0.2) (layer B.Cu) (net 25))
 (segment (start 63.6524 30.988) (end 62.8904 30.988) (width 0.2) (layer B.Cu) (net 25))
 (segment (start 66.04 31.623) (end 65.405 30.988) (width 0.2) (layer F.Cu) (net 24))
 (segment (start 66.04 33.808) (end 66.04 31.623) (width 0.2) (layer F.Cu) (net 24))
 (segment (start 66.3627 31.9203) (end 65.4304 30.988) (width 0.2) (layer B.Cu) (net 24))
 (segment (start 66.3627 35.008) (end 66.3627 31.9203) (width 0.2) (layer B.Cu) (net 24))
 (segment (start 67.31 33.808) (end 67.31 31.623) (width 0.2) (layer F.Cu) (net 23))
 (segment (start 67.31 31.623) (end 67.945 30.988) (width 0.2) (layer F.Cu) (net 23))
 (segment (start 67.0127 31.9457) (end 67.9704 30.988) (width 0.2) (layer B.Cu) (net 23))
 (segment (start 67.0127 35.008) (end 67.0127 31.9457) (width 0.2) (layer B.Cu) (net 23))
 (segment (start 69.635001 31.837999) (end 70.485 30.988) (width 0.2) (layer F.Cu) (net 20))
 (segment (start 68.58 32.893) (end 69.635001 31.837999) (width 0.2) (layer F.Cu) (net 20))
 (segment (start 68.58 33.808) (end 68.58 32.893) (width 0.2) (layer F.Cu) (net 20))
 (segment (start 69.7484 30.988) (end 70.5104 30.988) (width 0.2) (layer B.Cu) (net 20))
 (segment (start 67.6627 33.0737) (end 69.7484 30.988) (width 0.2) (layer B.Cu) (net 20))
 (segment (start 67.6627 35.008) (end 67.6627 33.0737) (width 0.2) (layer B.Cu) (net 20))
 (segment (start 72.2376 30.988) (end 73.025 30.988) (width 0.2) (layer F.Cu) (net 17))
 (segment (start 69.85 33.808) (end 69.85 33.3756) (width 0.2) (layer F.Cu) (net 17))
 (segment (start 69.85 33.3756) (end 72.2376 30.988) (width 0.2) (layer F.Cu) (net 17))
 (segment (start 71.9074 32.131) (end 73.0504 30.988) (width 0.2) (layer B.Cu) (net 17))
 (segment (start 68.3127 33.3127) (end 69.4944 32.131) (width 0.2) (layer B.Cu) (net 17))
 (segment (start 68.3127 35.008) (end 68.3127 33.3127) (width 0.2) (layer B.Cu) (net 17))
 (segment (start 69.4944 32.131) (end 71.9074 32.131) (width 0.2) (layer B.Cu) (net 17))
 (segment (start 68.9627 33.5517) (end 69.8754 32.639) (width 0.2) (layer B.Cu) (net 16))
 (segment (start 68.9627 35.008) (end 68.9627 33.5517) (width 0.2) (layer B.Cu) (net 16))
 (segment (start 73.9394 32.639) (end 75.5904 30.988) (width 0.2) (layer B.Cu) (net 16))
 (segment (start 69.8754 32.639) (end 73.9394 32.639) (width 0.2) (layer B.Cu) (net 16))
 (segment (start 74.715001 31.837999) (end 75.565 30.988) (width 0.2) (layer F.Cu) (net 16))
 (segment (start 74.422 32.131) (end 74.715001 31.837999) (width 0.2) (layer F.Cu) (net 16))
 (segment (start 71.7296 32.131) (end 74.422 32.131) (width 0.2) (layer F.Cu) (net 16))
 (segment (start 71.12 33.808) (end 71.12 32.7406) (width 0.2) (layer F.Cu) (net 16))
 (segment (start 71.12 32.7406) (end 71.7296 32.131) (width 0.2) (layer F.Cu) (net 16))
 (segment (start 72.898 32.4866) (end 76.6064 32.4866) (width 0.2) (layer F.Cu) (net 15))
 (segment (start 72.39 33.808) (end 72.39 32.9946) (width 0.2) (layer F.Cu) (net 15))
 (segment (start 72.39 32.9946) (end 72.898 32.4866) (width 0.2) (layer F.Cu) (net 15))
 (segment (start 76.6064 32.4866) (end 77.255001 31.837999) (width 0.2) (layer F.Cu) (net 15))
 (segment (start 77.255001 31.837999) (end 78.105 30.988) (width 0.2) (layer F.Cu) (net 15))
 (segment (start 69.6127 35.008) (end 69.6127 33.7907) (width 0.2) (layer B.Cu) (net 15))
 (segment (start 70.2564 33.147) (end 75.9714 33.147) (width 0.2) (layer B.Cu) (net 15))
 (segment (start 75.9714 33.147) (end 78.1304 30.988) (width 0.2) (layer B.Cu) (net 15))
 (segment (start 69.6127 33.7907) (end 70.2564 33.147) (width 0.2) (layer B.Cu) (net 15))
 (via (at 77.978 34.925) (size 0.8) (drill 0.4) (layers F.Cu B.Cu) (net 19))
 (segment (start 70.2627 35.008) (end 70.2627 33.933) (width 0.2) (layer B.Cu) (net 19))
 (segment (start 70.2627 33.933) (end 70.5407 33.655) (width 0.2) (layer B.Cu) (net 19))
 (segment (start 70.5407 33.655) (end 78.0034 33.655) (width 0.2) (layer B.Cu) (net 19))
 (segment (start 78.0034 33.655) (end 80.6704 30.988) (width 0.2) (layer B.Cu) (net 19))
 (segment (start 77.978 33.6804) (end 78.0034 33.655) (width 0.2) (layer B.Cu) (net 19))
 (segment (start 77.978 34.925) (end 77.978 33.6804) (width 0.2) (layer B.Cu) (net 19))
 (segment (start 77.978 37.719) (end 77.978 34.925) (width 0.2) (layer F.Cu) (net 19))
 (segment (start 77.47 38.227) (end 77.978 37.719) (width 0.2) (layer F.Cu) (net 19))
 (segment (start 74.168 38.227) (end 77.47 38.227) (width 0.2) (layer F.Cu) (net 19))
 (segment (start 73.66 33.808) (end 73.66 37.719) (width 0.2) (layer F.Cu) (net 19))
 (segment (start 73.66 37.719) (end 74.168 38.227) (width 0.2) (layer F.Cu) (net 19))
 (segment (start 74.93 33.808) (end 80.365 33.808) (width 0.2) (layer F.Cu) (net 18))
 (segment (start 80.365 33.808) (end 83.185 30.988) (width 0.2) (layer F.Cu) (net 18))
 (segment (start 78.0034 36.195) (end 83.2104 30.988) (width 0.2) (layer B.Cu) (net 18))
 (segment (start 70.9127 35.008) (end 72.0997 36.195) (width 0.2) (layer B.Cu) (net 18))
 (segment (start 72.0997 36.195) (end 78.0034 36.195) (width 0.2) (layer B.Cu) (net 18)))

